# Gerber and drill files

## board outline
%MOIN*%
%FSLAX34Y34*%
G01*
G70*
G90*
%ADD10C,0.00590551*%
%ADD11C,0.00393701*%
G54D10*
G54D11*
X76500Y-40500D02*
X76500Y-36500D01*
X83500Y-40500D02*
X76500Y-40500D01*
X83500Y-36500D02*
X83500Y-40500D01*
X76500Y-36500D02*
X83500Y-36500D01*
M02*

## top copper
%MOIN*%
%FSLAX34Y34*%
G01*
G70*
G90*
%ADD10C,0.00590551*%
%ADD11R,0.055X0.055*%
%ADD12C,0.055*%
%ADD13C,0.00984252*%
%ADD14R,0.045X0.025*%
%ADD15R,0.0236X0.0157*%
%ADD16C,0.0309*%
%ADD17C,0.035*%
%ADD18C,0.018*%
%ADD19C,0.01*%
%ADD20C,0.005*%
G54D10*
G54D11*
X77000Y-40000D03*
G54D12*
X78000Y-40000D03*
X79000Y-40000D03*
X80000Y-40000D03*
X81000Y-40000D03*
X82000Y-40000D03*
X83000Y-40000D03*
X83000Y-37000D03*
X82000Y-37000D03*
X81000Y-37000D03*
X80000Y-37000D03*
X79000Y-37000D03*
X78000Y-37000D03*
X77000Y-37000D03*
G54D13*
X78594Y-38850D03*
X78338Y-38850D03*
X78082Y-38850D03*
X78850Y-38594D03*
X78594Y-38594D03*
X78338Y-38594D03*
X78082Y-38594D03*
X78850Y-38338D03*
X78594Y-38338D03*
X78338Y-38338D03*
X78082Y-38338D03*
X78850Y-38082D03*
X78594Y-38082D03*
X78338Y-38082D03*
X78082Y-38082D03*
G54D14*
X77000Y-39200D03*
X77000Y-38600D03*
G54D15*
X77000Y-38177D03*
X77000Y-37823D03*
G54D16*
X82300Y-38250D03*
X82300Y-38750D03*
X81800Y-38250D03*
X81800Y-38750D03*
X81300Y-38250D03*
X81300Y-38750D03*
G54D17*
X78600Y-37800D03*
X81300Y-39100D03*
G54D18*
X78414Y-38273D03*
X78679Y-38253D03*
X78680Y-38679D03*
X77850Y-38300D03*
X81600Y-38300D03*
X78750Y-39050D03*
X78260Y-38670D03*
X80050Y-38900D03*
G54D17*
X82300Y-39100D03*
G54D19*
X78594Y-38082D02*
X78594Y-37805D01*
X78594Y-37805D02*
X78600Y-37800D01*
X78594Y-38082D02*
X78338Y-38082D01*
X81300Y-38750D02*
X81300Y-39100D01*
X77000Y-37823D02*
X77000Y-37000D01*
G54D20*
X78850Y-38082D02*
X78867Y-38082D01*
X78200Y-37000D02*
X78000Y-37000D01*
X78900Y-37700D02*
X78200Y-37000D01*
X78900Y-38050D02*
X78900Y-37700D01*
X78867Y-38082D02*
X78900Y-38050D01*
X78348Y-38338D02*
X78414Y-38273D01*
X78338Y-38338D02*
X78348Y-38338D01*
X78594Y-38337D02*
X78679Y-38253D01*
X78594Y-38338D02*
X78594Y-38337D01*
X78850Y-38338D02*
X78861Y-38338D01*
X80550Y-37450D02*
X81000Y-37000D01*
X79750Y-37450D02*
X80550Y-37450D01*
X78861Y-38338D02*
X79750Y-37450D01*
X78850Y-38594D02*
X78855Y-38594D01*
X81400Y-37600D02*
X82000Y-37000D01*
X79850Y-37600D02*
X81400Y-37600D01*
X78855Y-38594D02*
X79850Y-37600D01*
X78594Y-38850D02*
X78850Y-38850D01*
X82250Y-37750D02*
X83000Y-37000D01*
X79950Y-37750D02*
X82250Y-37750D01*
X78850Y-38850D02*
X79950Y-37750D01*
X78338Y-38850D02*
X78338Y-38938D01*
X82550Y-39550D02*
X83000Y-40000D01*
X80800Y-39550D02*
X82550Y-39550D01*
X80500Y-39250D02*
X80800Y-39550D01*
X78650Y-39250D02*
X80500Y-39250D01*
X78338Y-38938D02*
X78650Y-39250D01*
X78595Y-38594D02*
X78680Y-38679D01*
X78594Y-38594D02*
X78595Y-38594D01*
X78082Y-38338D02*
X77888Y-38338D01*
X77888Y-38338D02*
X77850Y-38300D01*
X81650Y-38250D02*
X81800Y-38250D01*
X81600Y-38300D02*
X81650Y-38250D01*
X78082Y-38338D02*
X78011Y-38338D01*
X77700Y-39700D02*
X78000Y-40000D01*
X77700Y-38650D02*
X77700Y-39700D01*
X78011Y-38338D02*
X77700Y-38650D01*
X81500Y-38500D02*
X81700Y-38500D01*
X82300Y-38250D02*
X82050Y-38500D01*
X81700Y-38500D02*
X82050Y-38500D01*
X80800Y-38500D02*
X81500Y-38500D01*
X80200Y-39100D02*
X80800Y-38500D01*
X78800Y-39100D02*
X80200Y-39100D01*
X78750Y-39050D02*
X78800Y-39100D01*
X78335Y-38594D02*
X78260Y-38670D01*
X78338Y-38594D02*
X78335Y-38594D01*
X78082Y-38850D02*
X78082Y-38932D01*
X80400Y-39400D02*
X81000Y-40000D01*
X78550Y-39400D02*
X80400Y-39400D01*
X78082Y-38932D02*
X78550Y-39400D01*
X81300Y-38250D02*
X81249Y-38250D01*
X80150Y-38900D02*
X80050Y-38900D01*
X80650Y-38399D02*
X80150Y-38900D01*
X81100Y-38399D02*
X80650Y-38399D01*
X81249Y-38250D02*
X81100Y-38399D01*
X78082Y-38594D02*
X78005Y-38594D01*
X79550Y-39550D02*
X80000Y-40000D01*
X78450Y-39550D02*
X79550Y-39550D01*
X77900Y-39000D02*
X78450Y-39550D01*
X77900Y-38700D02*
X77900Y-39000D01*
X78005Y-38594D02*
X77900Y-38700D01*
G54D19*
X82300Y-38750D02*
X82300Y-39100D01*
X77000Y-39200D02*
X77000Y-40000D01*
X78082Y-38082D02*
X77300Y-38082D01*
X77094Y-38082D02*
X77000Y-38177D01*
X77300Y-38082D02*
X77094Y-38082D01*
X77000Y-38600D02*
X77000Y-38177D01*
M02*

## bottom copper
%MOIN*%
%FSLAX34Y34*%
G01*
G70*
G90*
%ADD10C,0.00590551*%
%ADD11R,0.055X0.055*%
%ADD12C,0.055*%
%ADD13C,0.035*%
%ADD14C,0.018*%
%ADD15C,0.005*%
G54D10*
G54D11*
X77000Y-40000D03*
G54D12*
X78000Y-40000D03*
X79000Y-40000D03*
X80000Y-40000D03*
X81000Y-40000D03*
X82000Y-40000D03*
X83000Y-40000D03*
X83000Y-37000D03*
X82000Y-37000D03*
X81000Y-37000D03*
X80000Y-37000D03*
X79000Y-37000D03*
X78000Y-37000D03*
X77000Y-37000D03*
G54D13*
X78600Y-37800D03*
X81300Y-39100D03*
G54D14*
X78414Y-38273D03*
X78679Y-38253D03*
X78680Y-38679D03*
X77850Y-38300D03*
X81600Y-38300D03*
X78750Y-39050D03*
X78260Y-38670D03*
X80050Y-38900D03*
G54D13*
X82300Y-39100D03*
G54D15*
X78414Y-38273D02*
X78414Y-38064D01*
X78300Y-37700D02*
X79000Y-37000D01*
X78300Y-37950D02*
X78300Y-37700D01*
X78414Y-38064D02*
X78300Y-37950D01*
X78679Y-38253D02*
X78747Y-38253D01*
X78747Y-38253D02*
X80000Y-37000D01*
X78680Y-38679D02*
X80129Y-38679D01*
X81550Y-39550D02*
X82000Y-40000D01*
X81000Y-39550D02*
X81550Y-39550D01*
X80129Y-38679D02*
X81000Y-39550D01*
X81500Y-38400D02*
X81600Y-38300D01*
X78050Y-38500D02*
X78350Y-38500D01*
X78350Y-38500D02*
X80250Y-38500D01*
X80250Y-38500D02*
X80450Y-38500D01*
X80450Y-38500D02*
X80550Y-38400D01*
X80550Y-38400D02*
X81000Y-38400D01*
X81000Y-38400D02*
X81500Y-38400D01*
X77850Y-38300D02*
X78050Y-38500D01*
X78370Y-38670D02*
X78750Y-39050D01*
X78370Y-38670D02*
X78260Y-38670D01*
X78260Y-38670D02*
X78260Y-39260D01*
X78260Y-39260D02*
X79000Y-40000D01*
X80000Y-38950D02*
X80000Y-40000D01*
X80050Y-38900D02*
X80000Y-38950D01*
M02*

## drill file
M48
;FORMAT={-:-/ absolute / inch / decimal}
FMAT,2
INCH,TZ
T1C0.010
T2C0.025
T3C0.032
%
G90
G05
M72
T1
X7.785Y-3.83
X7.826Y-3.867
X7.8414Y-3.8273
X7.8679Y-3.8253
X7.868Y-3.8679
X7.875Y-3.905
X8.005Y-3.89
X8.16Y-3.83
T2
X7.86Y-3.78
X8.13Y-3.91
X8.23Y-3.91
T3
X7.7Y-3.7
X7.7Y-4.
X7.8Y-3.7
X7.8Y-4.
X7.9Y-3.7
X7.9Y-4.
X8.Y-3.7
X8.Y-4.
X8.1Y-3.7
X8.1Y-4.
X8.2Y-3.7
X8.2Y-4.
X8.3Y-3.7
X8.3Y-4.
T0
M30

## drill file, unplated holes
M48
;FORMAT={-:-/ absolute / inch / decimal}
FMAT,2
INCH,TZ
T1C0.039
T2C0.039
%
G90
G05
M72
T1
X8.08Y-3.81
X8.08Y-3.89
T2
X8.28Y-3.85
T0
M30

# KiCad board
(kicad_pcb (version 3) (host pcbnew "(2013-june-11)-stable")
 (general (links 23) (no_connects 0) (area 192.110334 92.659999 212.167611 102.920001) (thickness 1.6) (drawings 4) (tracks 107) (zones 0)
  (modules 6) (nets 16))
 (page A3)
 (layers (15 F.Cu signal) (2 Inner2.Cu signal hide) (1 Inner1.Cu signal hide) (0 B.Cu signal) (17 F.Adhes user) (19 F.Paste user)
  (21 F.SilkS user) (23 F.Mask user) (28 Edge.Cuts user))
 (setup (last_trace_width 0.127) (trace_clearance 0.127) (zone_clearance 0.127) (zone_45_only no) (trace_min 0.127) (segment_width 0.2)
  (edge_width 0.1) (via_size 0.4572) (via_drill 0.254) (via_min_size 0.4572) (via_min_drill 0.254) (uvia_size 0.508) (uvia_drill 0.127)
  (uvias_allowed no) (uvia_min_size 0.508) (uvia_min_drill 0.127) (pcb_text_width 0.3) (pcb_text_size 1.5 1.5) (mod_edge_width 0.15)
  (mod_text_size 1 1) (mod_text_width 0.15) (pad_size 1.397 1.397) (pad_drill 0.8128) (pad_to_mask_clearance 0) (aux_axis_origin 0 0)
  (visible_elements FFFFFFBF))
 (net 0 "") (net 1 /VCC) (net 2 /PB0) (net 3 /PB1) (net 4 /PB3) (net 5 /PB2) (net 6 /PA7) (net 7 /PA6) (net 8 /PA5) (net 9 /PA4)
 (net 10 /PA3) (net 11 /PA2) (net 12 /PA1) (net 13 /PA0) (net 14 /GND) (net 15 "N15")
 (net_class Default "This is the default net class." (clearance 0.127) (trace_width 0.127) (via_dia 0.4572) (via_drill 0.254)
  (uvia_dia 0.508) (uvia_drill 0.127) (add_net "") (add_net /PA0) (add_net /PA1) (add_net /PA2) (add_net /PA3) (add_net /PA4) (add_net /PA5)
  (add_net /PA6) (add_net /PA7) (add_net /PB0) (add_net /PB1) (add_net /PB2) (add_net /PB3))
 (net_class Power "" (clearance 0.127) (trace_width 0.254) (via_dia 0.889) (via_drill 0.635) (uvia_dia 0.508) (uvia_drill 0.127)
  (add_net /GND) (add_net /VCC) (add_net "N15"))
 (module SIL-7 (layer F.Cu) (at 203.2 101.6)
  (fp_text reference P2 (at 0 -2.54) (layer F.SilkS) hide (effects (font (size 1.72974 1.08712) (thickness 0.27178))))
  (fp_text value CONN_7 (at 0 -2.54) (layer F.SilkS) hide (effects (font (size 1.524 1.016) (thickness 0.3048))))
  (pad 1 thru_hole rect (at -7.62 0) (size 1.397 1.397) (drill 0.8128) (layers *.Cu *.Mask F.SilkS) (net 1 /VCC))
  (pad 2 thru_hole circle (at -5.08 0) (size 1.397 1.397) (drill 0.8128) (layers *.Cu *.SilkS *.Mask) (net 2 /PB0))
  (pad 3 thru_hole circle (at -2.54 0) (size 1.397 1.397) (drill 0.8128) (layers *.Cu *.SilkS *.Mask) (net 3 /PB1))
  (pad 4 thru_hole circle (at 0 0) (size 1.397 1.397) (drill 0.8128) (layers *.Cu *.SilkS *.Mask) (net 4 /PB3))
  (pad 5 thru_hole circle (at 2.54 0) (size 1.397 1.397) (drill 0.8128) (layers *.Cu *.SilkS *.Mask) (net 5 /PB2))
  (pad 6 thru_hole circle (at 5.08 0) (size 1.397 1.397) (drill 0.8128) (layers *.Cu *.SilkS *.Mask) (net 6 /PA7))
  (pad 7 thru_hole circle (at 7.62 0) (size 1.397 1.397) (drill 0.8128) (layers *.Cu *.SilkS *.Mask) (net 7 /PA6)))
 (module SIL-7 (layer F.Cu) (at 203.2 93.98 180)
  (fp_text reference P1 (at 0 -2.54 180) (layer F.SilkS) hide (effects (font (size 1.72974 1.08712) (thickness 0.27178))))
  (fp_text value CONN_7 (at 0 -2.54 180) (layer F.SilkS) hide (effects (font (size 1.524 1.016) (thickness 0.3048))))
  (pad 1 thru_hole circle (at -7.62 0 180) (size 1.397 1.397) (drill 0.8128) (layers *.Cu *.Mask F.SilkS) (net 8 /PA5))
  (pad 2 thru_hole circle (at -5.08 0 180) (size 1.397 1.397) (drill 0.8128) (layers *.Cu *.SilkS *.Mask) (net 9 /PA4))
  (pad 3 thru_hole circle (at -2.54 0 180) (size 1.397 1.397) (drill 0.8128) (layers *.Cu *.SilkS *.Mask) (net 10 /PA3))
  (pad 4 thru_hole circle (at 0 0 180) (size 1.397 1.397) (drill 0.8128) (layers *.Cu *.SilkS *.Mask) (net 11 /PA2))
  (pad 5 thru_hole circle (at 2.54 0 180) (size 1.397 1.397) (drill 0.8128) (layers *.Cu *.SilkS *.Mask) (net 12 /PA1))
  (pad 6 thru_hole circle (at 5.08 0 180) (size 1.397 1.397) (drill 0.8128) (layers *.Cu *.SilkS *.Mask) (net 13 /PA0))
  (pad 7 thru_hole circle (at 7.62 0 180) (size 1.397 1.397) (drill 0.8128) (layers *.Cu *.SilkS *.Mask) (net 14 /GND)))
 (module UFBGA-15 (layer F.Cu) (at 200.279 98.679 180) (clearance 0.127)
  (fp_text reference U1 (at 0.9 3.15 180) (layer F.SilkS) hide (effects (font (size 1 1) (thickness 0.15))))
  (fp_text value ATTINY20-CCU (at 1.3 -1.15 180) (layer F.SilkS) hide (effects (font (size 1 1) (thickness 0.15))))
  (pad A2 smd circle (at 0.65 0 180) (size 0.25 0.25) (layers F.Cu F.Paste F.Mask) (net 8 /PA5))
  (pad A3 smd circle (at 1.3 0 180) (size 0.25 0.25) (layers F.Cu F.Paste F.Mask) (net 7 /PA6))
  (pad A4 smd circle (at 1.95 0 180) (size 0.25 0.25) (layers F.Cu F.Paste F.Mask) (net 5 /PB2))
  (pad B1 smd circle (at 0 0.65 180) (size 0.25 0.25) (layers F.Cu F.Paste F.Mask) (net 9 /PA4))
  (pad B2 smd circle (at 0.65 0.65 180) (size 0.25 0.25) (layers F.Cu F.Paste F.Mask) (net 6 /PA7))
  (pad B3 smd circle (at 1.3 0.65 180) (size 0.25 0.25) (layers F.Cu F.Paste F.Mask) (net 3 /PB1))
  (pad B4 smd circle (at 1.95 0.65 180) (size 0.25 0.25) (layers F.Cu F.Paste F.Mask) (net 4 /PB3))
  (pad C1 smd circle (at 0 1.3 180) (size 0.25 0.25) (layers F.Cu F.Paste F.Mask) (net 10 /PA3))
  (pad C2 smd circle (at 0.65 1.3 180) (size 0.25 0.25) (layers F.Cu F.Paste F.Mask) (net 11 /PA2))
  (pad C3 smd circle (at 1.3 1.3 180) (size 0.25 0.25) (layers F.Cu F.Paste F.Mask) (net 12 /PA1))
  (pad C4 smd circle (at 1.95 1.3 180) (size 0.25 0.25) (layers F.Cu F.Paste F.Mask) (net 2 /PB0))
  (pad D1 smd circle (at 0 1.95 180) (size 0.25 0.25) (layers F.Cu F.Paste F.Mask) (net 13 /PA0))
  (pad D2 smd circle (at 0.65 1.95 180) (size 0.25 0.25) (layers F.Cu F.Paste F.Mask) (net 14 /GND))
  (pad D3 smd circle (at 1.3 1.95 180) (size 0.25 0.25) (layers F.Cu F.Paste F.Mask) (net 14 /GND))
  (pad D4 smd circle (at 1.95 1.95 180) (size 0.25 0.25) (layers F.Cu F.Paste F.Mask) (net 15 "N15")))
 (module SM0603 (layer F.Cu) (at 195.58 98.806 90)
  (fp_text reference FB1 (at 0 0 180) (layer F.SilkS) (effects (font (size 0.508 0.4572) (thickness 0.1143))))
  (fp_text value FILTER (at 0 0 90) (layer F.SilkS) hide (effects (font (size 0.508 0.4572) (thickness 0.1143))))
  (pad 1 smd rect (at -0.762 0 90) (size 0.635 1.143) (layers F.Cu F.Paste F.Mask) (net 1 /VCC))
  (pad 2 smd rect (at 0.762 0 90) (size 0.635 1.143) (layers F.Cu F.Paste F.Mask) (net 15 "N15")))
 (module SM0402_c (layer F.Cu) (at 195.58 96.52 90)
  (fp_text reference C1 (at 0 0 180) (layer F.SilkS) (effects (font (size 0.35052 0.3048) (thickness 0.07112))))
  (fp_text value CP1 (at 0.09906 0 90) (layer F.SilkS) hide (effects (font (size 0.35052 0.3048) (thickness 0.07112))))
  (pad 1 smd rect (at -0.44958 0 90) (size 0.39878 0.59944) (layers F.Cu F.Paste F.Mask) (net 15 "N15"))
  (pad 2 smd rect (at 0.44958 0 90) (size 0.39878 0.59944) (layers F.Cu F.Paste F.Mask) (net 14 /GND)))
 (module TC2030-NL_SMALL (layer F.Cu) (at 207.772 97.79 180) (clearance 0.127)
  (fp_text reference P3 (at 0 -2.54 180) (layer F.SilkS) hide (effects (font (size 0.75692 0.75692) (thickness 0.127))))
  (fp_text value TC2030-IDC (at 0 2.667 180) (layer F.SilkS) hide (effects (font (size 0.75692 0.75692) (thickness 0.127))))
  (pad 1 connect circle (at -1.27 0.635 180) (size 0.78486 0.78486) (layers F.Cu F.Mask) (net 3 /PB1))
  (pad 2 connect circle (at -1.27 -0.635 180) (size 0.78486 0.78486) (layers F.Cu F.Mask) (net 1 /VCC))
  (pad 3 connect circle (at 0 0.635 180) (size 0.78486 0.78486) (layers F.Cu F.Mask) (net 2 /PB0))
  (pad 4 connect circle (at 0 -0.635 180) (size 0.78486 0.78486) (layers F.Cu F.Mask))
  (pad 5 connect circle (at 1.27 0.635 180) (size 0.78486 0.78486) (layers F.Cu F.Mask) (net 4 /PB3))
  (pad 6 connect circle (at 1.27 -0.635 180) (size 0.78486 0.78486) (layers F.Cu F.Mask) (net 14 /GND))
  (pad "" np_thru_hole circle (at -2.54 0 180) (size 0.98806 0.98806) (drill 0.98806) (layers *.Cu *.Mask F.SilkS))
  (pad "" np_thru_hole circle (at 2.54 -1.016 180) (size 0.98552 0.98552) (drill 0.98552) (layers *.Cu *.Mask F.SilkS))
  (pad "" np_thru_hole circle (at 2.54 1.016 180) (size 0.98552 0.98552) (drill 0.98552) (layers *.Cu *.Mask F.SilkS)))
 (gr_line (start 194.31 102.87) (end 194.31 92.71) (angle 90) (layer Edge.Cuts) (width 0.1))
 (gr_line (start 212.09 102.87) (end 194.31 102.87) (angle 90) (layer Edge.Cuts) (width 0.1))
 (gr_line (start 212.09 92.71) (end 212.09 102.87) (angle 90) (layer Edge.Cuts) (width 0.1))
 (gr_line (start 194.31 92.71) (end 212.09 92.71) (angle 90) (layer Edge.Cuts) (width 0.1))
 (segment (start 199.629 96.729) (end 199.629 96.027) (width 0.254) (layer F.Cu) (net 14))
 (via (at 199.644 96.012) (size 0.889) (layers F.Cu B.Cu) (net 14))
 (segment (start 199.629 96.027) (end 199.644 96.012) (width 0.254) (layer F.Cu) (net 14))
 (segment (start 199.629 96.729) (end 198.979 96.729) (width 0.254) (layer F.Cu) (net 14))
 (segment (start 206.502 98.425) (end 206.502 99.314) (width 0.254) (layer F.Cu) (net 14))
 (via (at 206.502 99.314) (size 0.889) (layers F.Cu B.Cu) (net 14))
 (segment (start 195.58 96.07042) (end 195.58 93.98) (width 0.254) (layer F.Cu) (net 14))
 (segment (start 200.279 96.729) (end 200.324 96.729) (width 0.127) (layer F.Cu) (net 13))
 (segment (start 198.628 93.98) (end 198.12 93.98) (width 0.127) (layer F.Cu) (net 13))
 (segment (start 200.406 95.758) (end 198.628 93.98) (width 0.127) (layer F.Cu) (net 13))
 (segment (start 200.406 96.647) (end 200.406 95.758) (width 0.127) (layer F.Cu) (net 13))
 (segment (start 200.324 96.729) (end 200.406 96.647) (width 0.127) (layer F.Cu) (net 13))
 (segment (start 199.17156 97.21342) (end 199.17156 96.68256) (width 0.127) (layer B.Cu) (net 12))
 (segment (start 199.00598 97.379) (end 199.17156 97.21342) (width 0.127) (layer F.Cu) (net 12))
 (via (at 199.17156 97.21342) (size 0.4572) (layers F.Cu B.Cu) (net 12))
 (segment (start 198.979 97.379) (end 199.00598 97.379) (width 0.127) (layer F.Cu) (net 12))
 (segment (start 198.882 95.758) (end 200.66 93.98) (width 0.127) (layer B.Cu) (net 12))
 (segment (start 198.882 96.393) (end 198.882 95.758) (width 0.127) (layer B.Cu) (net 12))
 (segment (start 199.17156 96.68256) (end 198.882 96.393) (width 0.127) (layer B.Cu) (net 12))
 (segment (start 199.84466 97.16262) (end 200.01738 97.16262) (width 0.127) (layer B.Cu) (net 11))
 (segment (start 199.629 97.37828) (end 199.84466 97.16262) (width 0.127) (layer F.Cu) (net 11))
 (via (at 199.84466 97.16262) (size 0.4572) (layers F.Cu B.Cu) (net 11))
 (segment (start 199.629 97.379) (end 199.629 97.37828) (width 0.127) (layer F.Cu) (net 11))
 (segment (start 200.01738 97.16262) (end 203.2 93.98) (width 0.127) (layer B.Cu) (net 11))
 (segment (start 200.279 97.379) (end 200.309 97.379) (width 0.127) (layer F.Cu) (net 10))
 (segment (start 204.597 95.123) (end 205.74 93.98) (width 0.127) (layer F.Cu) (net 10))
 (segment (start 202.565 95.123) (end 204.597 95.123) (width 0.127) (layer F.Cu) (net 10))
 (segment (start 200.309 97.379) (end 202.565 95.123) (width 0.127) (layer F.Cu) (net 10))
 (segment (start 200.279 98.029) (end 200.294 98.029) (width 0.127) (layer F.Cu) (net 9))
 (segment (start 206.756 95.504) (end 208.28 93.98) (width 0.127) (layer F.Cu) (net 9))
 (segment (start 202.819 95.504) (end 206.756 95.504) (width 0.127) (layer F.Cu) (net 9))
 (segment (start 200.294 98.029) (end 202.819 95.504) (width 0.127) (layer F.Cu) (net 9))
 (segment (start 199.629 98.679) (end 200.279 98.679) (width 0.127) (layer F.Cu) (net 8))
 (segment (start 208.915 95.885) (end 210.82 93.98) (width 0.127) (layer F.Cu) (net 8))
 (segment (start 203.073 95.885) (end 208.915 95.885) (width 0.127) (layer F.Cu) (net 8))
 (segment (start 200.279 98.679) (end 203.073 95.885) (width 0.127) (layer F.Cu) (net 8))
 (segment (start 198.979 98.679) (end 198.979 98.903) (width 0.127) (layer F.Cu) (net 7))
 (segment (start 209.677 100.457) (end 210.82 101.6) (width 0.127) (layer F.Cu) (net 7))
 (segment (start 205.232 100.457) (end 209.677 100.457) (width 0.127) (layer F.Cu) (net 7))
 (segment (start 204.47 99.695) (end 205.232 100.457) (width 0.127) (layer F.Cu) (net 7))
 (segment (start 199.771 99.695) (end 204.47 99.695) (width 0.127) (layer F.Cu) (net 7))
 (segment (start 198.979 98.903) (end 199.771 99.695) (width 0.127) (layer F.Cu) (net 7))
 (segment (start 199.8472 98.24466) (end 203.52766 98.24466) (width 0.127) (layer B.Cu) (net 6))
 (segment (start 199.63154 98.029) (end 199.8472 98.24466) (width 0.127) (layer F.Cu) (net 6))
 (via (at 199.8472 98.24466) (size 0.4572) (layers F.Cu B.Cu) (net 6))
 (segment (start 199.629 98.029) (end 199.63154 98.029) (width 0.127) (layer F.Cu) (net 6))
 (segment (start 207.137 100.457) (end 208.28 101.6) (width 0.127) (layer B.Cu) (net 6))
 (segment (start 205.74 100.457) (end 207.137 100.457) (width 0.127) (layer B.Cu) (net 6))
 (segment (start 203.52766 98.24466) (end 205.74 100.457) (width 0.127) (layer B.Cu) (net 6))
 (segment (start 207.01 97.536) (end 207.264 97.282) (width 0.127) (layer B.Cu) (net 2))
 (segment (start 198.247 97.79) (end 199.009 97.79) (width 0.127) (layer B.Cu) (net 2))
 (segment (start 199.009 97.79) (end 203.835 97.79) (width 0.127) (layer B.Cu) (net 2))
 (segment (start 203.835 97.79) (end 204.343 97.79) (width 0.127) (layer B.Cu) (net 2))
 (segment (start 204.343 97.79) (end 204.597 97.536) (width 0.127) (layer B.Cu) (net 2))
 (segment (start 204.597 97.536) (end 205.74 97.536) (width 0.127) (layer B.Cu) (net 2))
 (segment (start 205.74 97.536) (end 207.01 97.536) (width 0.127) (layer B.Cu) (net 2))
 (segment (start 198.329 97.379) (end 197.836 97.379) (width 0.127) (layer F.Cu) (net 2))
 (via (at 197.739 97.282) (size 0.4572) (layers F.Cu B.Cu) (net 2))
 (segment (start 197.836 97.379) (end 197.739 97.282) (width 0.127) (layer F.Cu) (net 2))
 (segment (start 197.739 97.282) (end 198.247 97.79) (width 0.127) (layer B.Cu) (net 2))
 (segment (start 207.391 97.155) (end 207.772 97.155) (width 0.127) (layer F.Cu) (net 2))
 (segment (start 207.264 97.282) (end 207.391 97.155) (width 0.127) (layer F.Cu) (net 2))
 (via (at 207.264 97.282) (size 0.4572) (layers F.Cu B.Cu) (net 2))
 (segment (start 198.329 97.379) (end 198.15 97.379) (width 0.127) (layer F.Cu) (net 2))
 (segment (start 197.358 100.838) (end 198.12 101.6) (width 0.127) (layer F.Cu) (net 2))
 (segment (start 197.358 98.171) (end 197.358 100.838) (width 0.127) (layer F.Cu) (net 2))
 (segment (start 198.15 97.379) (end 197.358 98.171) (width 0.127) (layer F.Cu) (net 2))
 (segment (start 207.01 97.79) (end 207.518 97.79) (width 0.127) (layer F.Cu) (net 3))
 (segment (start 209.042 97.155) (end 208.407 97.79) (width 0.127) (layer F.Cu) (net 3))
 (segment (start 207.518 97.79) (end 208.407 97.79) (width 0.127) (layer F.Cu) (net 3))
 (segment (start 205.232 97.79) (end 207.01 97.79) (width 0.127) (layer F.Cu) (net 3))
 (segment (start 203.708 99.314) (end 205.232 97.79) (width 0.127) (layer F.Cu) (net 3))
 (segment (start 200.152 99.314) (end 203.708 99.314) (width 0.127) (layer F.Cu) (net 3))
 (segment (start 200.025 99.187) (end 200.152 99.314) (width 0.127) (layer F.Cu) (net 3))
 (via (at 200.025 99.187) (size 0.4572) (layers F.Cu B.Cu) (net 3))
 (segment (start 199.0598 98.2218) (end 200.025 99.187) (width 0.127) (layer B.Cu) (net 3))
 (segment (start 199.0598 98.2218) (end 198.7804 98.2218) (width 0.127) (layer B.Cu) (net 3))
 (segment (start 198.7804 98.2218) (end 198.7804 99.7204) (width 0.127) (layer B.Cu) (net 3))
 (segment (start 198.9732 98.029) (end 198.7804 98.2218) (width 0.127) (layer F.Cu) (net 3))
 (via (at 198.7804 98.2218) (size 0.4572) (layers F.Cu B.Cu) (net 3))
 (segment (start 198.979 98.029) (end 198.9732 98.029) (width 0.127) (layer F.Cu) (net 3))
 (segment (start 198.7804 99.7204) (end 200.66 101.6) (width 0.127) (layer B.Cu) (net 3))
 (segment (start 198.329 98.679) (end 198.329 98.888) (width 0.127) (layer F.Cu) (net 5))
 (segment (start 204.216 100.076) (end 205.74 101.6) (width 0.127) (layer F.Cu) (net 5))
 (segment (start 199.517 100.076) (end 204.216 100.076) (width 0.127) (layer F.Cu) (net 5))
 (segment (start 198.329 98.888) (end 199.517 100.076) (width 0.127) (layer F.Cu) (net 5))
 (segment (start 206.502 97.155) (end 206.374998 97.155) (width 0.127) (layer F.Cu) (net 4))
 (segment (start 203.2 98.933) (end 203.2 101.6) (width 0.127) (layer B.Cu) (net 4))
 (segment (start 203.327 98.806) (end 203.2 98.933) (width 0.127) (layer B.Cu) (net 4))
 (via (at 203.327 98.806) (size 0.4572) (layers F.Cu B.Cu) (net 4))
 (segment (start 203.581 98.806) (end 203.327 98.806) (width 0.127) (layer F.Cu) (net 4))
 (segment (start 204.851002 97.535998) (end 203.581 98.806) (width 0.127) (layer F.Cu) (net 4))
 (segment (start 205.994 97.535998) (end 204.851002 97.535998) (width 0.127) (layer F.Cu) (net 4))
 (segment (start 206.374998 97.155) (end 205.994 97.535998) (width 0.127) (layer F.Cu) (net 4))
 (segment (start 198.329 98.029) (end 198.135 98.029) (width 0.127) (layer F.Cu) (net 4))
 (segment (start 202.057 100.457) (end 203.2 101.6) (width 0.127) (layer F.Cu) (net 4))
 (segment (start 199.263 100.457) (end 202.057 100.457) (width 0.127) (layer F.Cu) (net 4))
 (segment (start 197.866 99.06) (end 199.263 100.457) (width 0.127) (layer F.Cu) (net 4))
 (segment (start 197.866 98.298) (end 197.866 99.06) (width 0.127) (layer F.Cu) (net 4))
 (segment (start 198.135 98.029) (end 197.866 98.298) (width 0.127) (layer F.Cu) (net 4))
 (segment (start 209.042 98.425) (end 209.042 99.314) (width 0.254) (layer F.Cu) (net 1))
 (via (at 209.042 99.314) (size 0.889) (layers F.Cu B.Cu) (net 1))
 (segment (start 195.58 99.568) (end 195.58 101.6) (width 0.254) (layer F.Cu) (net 1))
 (segment (start 198.329 96.729) (end 196.342 96.729) (width 0.254) (layer F.Cu) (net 15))
 (segment (start 195.82058 96.729) (end 195.58 96.96958) (width 0.254) (layer F.Cu) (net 15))
 (segment (start 196.342 96.729) (end 195.82058 96.729) (width 0.254) (layer F.Cu) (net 15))
 (segment (start 195.58 98.044) (end 195.58 96.96958) (width 0.254) (layer F.Cu) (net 15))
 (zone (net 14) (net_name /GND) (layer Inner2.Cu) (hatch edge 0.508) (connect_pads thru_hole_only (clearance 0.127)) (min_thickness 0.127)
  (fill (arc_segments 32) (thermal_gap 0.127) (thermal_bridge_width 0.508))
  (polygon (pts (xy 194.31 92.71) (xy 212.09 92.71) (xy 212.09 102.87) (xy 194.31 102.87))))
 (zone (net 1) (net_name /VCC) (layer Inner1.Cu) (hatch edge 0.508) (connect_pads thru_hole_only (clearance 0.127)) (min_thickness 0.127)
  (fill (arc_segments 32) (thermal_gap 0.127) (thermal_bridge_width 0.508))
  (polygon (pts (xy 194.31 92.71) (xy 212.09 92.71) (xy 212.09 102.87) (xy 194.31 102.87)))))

